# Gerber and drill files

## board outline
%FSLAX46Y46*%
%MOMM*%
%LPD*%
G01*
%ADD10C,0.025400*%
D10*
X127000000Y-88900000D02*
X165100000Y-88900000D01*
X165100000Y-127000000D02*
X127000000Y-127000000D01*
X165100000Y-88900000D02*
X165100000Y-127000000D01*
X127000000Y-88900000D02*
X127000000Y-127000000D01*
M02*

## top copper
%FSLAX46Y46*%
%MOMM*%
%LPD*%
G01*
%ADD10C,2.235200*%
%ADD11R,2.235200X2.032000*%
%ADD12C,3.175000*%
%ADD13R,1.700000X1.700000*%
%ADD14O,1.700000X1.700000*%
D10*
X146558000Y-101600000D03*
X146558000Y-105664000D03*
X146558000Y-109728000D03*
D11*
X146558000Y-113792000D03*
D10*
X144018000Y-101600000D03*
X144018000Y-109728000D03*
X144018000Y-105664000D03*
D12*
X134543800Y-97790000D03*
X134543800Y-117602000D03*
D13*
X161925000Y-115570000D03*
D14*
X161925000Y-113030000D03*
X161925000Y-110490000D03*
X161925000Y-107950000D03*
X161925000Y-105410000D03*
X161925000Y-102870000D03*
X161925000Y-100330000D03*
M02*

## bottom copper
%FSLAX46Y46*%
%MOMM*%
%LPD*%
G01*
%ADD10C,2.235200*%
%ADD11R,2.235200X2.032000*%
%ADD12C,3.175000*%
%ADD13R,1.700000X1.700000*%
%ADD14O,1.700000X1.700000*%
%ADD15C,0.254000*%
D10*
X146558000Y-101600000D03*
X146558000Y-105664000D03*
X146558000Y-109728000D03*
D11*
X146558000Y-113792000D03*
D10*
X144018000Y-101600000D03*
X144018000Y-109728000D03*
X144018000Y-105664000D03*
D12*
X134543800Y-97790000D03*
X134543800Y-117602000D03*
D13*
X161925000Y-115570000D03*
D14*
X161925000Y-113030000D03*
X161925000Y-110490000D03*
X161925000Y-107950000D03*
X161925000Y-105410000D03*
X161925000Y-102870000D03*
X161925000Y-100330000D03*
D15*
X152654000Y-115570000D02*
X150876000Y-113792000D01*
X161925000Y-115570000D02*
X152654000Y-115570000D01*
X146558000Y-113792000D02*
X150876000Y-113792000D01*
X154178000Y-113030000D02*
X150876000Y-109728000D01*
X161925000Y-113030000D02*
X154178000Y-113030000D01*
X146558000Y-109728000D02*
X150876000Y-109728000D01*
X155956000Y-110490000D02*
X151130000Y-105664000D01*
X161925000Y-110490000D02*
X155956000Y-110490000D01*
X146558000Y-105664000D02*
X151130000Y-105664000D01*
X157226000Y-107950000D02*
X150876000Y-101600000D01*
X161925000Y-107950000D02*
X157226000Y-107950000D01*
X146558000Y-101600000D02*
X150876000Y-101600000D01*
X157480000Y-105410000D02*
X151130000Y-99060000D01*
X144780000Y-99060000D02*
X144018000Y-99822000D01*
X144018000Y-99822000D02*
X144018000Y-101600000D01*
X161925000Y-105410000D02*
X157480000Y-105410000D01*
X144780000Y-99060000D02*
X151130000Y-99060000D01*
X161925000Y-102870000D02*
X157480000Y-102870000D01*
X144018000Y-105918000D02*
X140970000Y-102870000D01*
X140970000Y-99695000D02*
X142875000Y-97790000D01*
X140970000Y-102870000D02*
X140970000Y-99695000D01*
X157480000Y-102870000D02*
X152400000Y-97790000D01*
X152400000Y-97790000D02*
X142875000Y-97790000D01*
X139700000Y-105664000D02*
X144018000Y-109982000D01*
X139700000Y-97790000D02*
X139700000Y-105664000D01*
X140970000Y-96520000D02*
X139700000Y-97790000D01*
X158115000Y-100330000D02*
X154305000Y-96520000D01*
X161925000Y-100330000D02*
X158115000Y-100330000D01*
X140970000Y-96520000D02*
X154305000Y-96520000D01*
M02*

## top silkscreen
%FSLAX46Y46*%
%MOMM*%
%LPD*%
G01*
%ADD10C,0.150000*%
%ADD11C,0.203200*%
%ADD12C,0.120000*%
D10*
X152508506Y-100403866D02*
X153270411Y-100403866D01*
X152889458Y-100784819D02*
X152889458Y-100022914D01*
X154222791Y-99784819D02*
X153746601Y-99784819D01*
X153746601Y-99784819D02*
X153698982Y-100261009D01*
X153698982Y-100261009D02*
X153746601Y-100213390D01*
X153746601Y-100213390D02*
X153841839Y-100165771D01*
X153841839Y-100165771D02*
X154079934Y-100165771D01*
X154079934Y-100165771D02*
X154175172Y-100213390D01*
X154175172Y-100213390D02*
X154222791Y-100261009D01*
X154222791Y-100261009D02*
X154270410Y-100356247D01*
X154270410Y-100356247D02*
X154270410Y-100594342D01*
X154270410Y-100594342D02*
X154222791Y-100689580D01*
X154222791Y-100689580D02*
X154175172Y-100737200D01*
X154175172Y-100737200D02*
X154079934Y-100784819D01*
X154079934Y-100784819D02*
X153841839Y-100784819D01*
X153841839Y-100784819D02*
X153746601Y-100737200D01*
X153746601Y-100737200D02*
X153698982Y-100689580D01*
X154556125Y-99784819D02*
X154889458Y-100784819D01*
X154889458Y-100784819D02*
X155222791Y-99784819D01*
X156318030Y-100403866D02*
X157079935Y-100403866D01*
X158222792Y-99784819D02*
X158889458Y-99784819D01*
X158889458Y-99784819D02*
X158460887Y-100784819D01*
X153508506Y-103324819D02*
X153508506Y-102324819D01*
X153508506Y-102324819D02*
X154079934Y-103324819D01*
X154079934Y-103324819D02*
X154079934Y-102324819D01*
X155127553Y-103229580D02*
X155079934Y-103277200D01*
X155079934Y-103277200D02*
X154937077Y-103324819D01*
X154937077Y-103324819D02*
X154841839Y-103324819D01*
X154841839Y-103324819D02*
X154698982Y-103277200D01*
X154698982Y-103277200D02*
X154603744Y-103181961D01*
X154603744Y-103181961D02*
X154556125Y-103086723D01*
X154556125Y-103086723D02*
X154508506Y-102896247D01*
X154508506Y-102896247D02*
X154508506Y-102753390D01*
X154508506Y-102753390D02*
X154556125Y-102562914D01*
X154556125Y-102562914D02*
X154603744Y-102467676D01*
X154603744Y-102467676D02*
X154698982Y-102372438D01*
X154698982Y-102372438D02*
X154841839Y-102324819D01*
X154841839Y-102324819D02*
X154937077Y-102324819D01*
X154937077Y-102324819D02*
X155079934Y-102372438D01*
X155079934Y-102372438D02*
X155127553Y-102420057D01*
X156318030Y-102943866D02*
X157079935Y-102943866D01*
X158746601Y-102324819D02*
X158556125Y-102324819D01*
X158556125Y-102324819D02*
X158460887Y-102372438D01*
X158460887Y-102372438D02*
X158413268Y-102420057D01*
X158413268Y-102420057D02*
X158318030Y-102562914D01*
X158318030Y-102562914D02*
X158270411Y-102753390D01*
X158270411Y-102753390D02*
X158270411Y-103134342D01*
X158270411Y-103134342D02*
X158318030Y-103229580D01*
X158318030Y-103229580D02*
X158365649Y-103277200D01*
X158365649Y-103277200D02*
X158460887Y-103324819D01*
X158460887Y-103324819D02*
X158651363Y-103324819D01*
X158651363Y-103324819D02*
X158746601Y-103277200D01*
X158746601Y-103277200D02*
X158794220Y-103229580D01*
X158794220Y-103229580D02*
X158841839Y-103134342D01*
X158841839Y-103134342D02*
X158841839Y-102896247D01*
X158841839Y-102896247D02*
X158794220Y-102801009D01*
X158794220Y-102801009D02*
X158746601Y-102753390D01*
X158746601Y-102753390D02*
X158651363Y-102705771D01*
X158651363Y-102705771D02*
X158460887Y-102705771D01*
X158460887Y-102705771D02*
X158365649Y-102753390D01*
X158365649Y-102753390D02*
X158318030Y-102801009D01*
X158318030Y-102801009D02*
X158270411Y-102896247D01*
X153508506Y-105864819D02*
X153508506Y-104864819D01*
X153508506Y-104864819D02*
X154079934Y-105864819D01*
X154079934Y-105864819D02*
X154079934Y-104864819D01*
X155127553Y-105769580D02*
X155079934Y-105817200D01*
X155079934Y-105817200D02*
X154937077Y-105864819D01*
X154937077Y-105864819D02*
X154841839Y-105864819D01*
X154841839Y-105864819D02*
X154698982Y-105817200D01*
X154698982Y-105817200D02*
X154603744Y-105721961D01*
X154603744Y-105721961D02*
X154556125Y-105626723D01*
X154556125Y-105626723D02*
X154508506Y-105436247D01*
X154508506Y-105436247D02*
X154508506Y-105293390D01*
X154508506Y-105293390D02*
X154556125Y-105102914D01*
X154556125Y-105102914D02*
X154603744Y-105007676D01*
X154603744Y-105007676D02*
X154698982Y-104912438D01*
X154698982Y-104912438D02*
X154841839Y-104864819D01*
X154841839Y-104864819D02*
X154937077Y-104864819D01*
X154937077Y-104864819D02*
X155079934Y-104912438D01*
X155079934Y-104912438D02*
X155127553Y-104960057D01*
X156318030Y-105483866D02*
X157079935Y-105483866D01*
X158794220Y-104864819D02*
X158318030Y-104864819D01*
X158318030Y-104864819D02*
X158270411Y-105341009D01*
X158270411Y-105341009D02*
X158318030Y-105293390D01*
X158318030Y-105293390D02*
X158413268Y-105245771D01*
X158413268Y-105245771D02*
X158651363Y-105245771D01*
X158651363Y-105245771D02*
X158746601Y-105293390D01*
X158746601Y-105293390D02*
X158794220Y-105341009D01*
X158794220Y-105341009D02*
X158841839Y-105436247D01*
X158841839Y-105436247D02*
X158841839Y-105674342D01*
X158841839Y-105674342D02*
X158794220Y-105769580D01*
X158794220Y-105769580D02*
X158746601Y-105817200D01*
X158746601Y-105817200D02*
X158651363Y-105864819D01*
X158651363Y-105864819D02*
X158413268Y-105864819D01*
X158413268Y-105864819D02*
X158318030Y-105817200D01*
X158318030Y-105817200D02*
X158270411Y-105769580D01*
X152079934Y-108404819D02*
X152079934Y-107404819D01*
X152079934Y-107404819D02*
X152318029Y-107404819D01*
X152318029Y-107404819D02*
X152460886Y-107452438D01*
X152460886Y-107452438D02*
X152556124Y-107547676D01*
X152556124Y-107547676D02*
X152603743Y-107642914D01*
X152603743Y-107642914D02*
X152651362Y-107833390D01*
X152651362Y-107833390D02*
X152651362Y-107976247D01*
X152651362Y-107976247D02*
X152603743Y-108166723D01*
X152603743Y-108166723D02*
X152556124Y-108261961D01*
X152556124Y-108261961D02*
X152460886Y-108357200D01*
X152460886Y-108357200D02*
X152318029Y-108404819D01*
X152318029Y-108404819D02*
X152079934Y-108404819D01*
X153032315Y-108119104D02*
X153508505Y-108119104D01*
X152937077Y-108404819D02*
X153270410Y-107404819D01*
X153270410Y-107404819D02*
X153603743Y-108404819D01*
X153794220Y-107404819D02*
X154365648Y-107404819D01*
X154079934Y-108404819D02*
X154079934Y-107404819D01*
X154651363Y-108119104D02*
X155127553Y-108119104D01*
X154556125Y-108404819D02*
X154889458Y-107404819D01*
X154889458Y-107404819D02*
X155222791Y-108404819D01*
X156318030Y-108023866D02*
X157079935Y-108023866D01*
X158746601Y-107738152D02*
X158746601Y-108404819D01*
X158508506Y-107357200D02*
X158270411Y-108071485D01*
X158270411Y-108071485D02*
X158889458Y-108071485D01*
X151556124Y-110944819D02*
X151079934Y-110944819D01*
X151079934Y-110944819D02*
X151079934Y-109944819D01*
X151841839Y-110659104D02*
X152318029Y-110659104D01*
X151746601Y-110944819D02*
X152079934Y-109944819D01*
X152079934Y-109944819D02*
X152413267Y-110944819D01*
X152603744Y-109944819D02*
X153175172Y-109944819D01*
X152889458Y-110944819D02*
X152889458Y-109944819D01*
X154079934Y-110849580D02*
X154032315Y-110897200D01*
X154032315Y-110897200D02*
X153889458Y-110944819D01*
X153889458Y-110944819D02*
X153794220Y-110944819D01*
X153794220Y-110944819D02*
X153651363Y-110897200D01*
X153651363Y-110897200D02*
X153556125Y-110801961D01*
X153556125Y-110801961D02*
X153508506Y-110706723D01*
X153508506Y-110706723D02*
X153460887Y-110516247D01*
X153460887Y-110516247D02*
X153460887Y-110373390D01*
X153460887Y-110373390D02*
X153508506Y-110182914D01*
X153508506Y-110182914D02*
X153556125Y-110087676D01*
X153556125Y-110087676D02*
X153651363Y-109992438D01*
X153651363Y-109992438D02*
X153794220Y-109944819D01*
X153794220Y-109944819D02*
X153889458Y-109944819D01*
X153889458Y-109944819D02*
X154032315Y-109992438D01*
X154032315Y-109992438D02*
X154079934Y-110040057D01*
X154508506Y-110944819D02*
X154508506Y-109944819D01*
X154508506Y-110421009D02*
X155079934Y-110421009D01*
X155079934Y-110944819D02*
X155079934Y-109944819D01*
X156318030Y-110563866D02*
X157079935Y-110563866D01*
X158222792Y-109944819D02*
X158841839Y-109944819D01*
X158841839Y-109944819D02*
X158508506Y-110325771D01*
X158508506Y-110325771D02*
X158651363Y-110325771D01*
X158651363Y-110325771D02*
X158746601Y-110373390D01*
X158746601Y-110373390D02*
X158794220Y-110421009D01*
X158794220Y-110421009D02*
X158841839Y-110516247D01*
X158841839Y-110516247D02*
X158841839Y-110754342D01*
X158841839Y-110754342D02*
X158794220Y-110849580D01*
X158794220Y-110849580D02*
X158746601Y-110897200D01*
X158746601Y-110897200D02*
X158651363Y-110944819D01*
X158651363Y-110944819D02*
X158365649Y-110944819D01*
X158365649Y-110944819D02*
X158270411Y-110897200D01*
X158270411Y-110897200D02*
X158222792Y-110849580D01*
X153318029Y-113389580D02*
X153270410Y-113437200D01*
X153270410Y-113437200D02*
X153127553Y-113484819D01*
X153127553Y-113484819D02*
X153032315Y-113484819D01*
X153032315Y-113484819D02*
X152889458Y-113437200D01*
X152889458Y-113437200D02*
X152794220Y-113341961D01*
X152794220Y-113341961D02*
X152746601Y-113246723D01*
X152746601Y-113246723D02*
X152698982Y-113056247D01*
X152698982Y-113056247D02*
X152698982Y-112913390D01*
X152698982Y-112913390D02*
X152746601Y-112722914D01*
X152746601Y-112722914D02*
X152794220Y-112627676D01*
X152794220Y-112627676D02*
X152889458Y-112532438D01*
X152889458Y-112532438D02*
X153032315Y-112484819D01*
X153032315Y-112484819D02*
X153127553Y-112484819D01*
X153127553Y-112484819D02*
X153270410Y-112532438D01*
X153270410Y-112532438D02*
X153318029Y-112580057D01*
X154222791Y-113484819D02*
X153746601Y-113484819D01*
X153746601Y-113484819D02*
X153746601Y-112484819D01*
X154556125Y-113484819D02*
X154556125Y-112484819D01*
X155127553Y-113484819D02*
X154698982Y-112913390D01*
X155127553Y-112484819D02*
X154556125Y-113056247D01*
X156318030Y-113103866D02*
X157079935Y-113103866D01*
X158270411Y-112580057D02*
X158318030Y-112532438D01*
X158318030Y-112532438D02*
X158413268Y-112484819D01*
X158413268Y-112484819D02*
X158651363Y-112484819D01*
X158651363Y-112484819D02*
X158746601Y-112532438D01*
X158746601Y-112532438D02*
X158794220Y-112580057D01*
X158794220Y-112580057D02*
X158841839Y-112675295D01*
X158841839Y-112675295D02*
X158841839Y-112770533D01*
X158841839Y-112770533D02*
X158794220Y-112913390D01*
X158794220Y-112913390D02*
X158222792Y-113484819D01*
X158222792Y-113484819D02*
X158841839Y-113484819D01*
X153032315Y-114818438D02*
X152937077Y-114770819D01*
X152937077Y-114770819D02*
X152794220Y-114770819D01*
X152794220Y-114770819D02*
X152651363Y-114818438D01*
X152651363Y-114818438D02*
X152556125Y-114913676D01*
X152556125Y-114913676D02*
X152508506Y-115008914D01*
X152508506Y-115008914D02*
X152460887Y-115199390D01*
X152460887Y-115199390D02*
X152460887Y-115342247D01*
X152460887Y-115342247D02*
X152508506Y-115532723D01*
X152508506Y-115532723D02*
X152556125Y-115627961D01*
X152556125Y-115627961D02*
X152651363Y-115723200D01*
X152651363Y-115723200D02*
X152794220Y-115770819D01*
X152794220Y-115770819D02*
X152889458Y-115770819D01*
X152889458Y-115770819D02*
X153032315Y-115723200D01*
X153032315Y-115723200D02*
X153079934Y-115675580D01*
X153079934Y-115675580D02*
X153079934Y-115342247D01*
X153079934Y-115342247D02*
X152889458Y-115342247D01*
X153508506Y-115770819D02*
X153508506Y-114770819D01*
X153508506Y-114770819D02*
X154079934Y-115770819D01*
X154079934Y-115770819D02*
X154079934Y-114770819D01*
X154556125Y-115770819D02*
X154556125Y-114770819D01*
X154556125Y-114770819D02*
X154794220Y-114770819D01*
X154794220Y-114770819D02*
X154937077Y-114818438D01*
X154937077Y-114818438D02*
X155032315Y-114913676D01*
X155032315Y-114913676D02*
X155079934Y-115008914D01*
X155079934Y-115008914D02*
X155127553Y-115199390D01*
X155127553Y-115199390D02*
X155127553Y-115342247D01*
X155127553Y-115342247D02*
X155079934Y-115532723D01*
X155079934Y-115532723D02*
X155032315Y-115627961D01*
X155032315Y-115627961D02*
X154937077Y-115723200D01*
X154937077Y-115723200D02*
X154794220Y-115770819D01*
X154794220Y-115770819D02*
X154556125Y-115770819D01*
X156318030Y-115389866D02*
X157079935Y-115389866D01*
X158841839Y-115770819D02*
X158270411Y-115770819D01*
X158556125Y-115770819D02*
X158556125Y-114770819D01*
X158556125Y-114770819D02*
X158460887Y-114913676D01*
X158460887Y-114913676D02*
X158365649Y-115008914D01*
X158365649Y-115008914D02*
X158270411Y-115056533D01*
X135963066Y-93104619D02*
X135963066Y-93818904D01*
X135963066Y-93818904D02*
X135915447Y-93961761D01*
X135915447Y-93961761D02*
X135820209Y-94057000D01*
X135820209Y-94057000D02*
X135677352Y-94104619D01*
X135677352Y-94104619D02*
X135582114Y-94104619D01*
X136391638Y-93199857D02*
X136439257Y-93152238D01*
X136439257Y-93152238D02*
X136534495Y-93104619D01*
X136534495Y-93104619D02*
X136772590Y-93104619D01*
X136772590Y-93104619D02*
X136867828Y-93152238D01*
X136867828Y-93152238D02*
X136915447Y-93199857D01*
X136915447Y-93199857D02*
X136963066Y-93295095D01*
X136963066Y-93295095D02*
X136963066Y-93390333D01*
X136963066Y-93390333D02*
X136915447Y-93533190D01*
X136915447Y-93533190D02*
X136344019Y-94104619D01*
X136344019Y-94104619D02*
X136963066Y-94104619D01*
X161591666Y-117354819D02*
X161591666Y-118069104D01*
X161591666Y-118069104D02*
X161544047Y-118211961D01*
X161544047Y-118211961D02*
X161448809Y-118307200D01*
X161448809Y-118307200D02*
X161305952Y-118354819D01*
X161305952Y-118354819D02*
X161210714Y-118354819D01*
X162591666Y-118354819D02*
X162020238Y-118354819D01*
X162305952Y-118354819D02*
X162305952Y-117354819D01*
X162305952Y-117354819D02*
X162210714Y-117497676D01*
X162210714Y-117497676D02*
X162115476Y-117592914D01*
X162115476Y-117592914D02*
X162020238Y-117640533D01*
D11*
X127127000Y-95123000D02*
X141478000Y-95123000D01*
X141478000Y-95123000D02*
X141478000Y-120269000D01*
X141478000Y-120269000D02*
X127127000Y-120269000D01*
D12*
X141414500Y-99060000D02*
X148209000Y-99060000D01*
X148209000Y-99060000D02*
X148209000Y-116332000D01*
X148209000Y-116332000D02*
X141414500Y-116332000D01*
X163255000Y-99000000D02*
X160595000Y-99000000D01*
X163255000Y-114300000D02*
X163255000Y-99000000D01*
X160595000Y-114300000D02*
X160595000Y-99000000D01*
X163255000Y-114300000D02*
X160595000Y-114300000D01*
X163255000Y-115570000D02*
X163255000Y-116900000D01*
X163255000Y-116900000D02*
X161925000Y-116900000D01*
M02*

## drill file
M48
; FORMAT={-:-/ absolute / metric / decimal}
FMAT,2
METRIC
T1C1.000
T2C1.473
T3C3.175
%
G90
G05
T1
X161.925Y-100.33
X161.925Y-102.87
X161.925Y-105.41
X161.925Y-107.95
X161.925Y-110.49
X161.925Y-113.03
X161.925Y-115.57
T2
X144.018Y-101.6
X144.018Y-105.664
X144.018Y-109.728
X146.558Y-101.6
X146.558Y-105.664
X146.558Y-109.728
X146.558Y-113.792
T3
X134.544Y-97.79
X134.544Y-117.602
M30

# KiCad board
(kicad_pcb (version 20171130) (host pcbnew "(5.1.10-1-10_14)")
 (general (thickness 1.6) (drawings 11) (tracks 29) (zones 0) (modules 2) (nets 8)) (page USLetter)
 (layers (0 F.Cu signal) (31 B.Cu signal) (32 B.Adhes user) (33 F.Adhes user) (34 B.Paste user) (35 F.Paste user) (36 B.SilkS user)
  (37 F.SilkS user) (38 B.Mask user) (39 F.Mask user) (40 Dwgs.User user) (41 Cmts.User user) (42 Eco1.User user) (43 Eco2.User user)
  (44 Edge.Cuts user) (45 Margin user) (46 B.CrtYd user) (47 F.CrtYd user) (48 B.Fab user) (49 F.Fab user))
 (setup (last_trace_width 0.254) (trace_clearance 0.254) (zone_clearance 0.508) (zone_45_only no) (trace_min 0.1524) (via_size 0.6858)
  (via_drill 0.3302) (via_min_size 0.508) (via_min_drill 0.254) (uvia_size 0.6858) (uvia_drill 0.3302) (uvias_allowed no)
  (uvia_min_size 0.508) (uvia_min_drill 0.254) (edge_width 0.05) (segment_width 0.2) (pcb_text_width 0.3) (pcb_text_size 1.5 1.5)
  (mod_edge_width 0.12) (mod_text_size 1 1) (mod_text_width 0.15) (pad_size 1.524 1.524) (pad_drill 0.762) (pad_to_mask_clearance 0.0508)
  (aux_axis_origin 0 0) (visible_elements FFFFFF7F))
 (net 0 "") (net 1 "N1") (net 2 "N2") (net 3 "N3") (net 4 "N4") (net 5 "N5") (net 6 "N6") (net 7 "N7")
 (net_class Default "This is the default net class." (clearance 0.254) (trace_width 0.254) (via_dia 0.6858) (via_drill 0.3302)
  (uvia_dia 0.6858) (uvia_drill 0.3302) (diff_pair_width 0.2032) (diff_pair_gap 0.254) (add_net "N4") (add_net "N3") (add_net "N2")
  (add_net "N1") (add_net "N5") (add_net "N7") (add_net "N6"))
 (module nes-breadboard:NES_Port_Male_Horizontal (layer F.Cu) (at 147.574 107.696)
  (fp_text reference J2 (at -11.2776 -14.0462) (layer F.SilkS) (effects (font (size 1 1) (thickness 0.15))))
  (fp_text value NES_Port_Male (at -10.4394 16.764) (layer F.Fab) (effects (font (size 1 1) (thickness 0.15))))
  (fp_line (start -20.447 -12.573) (end -6.096 -12.573) (layer F.SilkS) (width 0.2032))
  (fp_line (start -6.096 -12.573) (end -6.096 12.573) (layer F.SilkS) (width 0.2032))
  (fp_line (start -6.096 12.573) (end -20.447 12.573) (layer F.SilkS) (width 0.2032))
  (fp_line (start -6.1595 -8.636) (end 0.635 -8.636) (layer F.SilkS) (width 0.12))
  (fp_line (start 0.635 -8.636) (end 0.635 8.636) (layer F.SilkS) (width 0.12))
  (fp_line (start 0.635 8.636) (end -6.1595 8.636) (layer F.SilkS) (width 0.12))
  (pad 4 thru_hole circle (at -1.016 -6.096) (size 2.2352 2.2352) (drill 1.4732) (layers *.Cu *.Mask) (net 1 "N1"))
  (pad 3 thru_hole circle (at -1.016 -2.032) (size 2.2352 2.2352) (drill 1.4732) (layers *.Cu *.Mask) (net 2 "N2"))
  (pad 2 thru_hole circle (at -1.016 2.032) (size 2.2352 2.2352) (drill 1.4732) (layers *.Cu *.Mask) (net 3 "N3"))
  (pad 1 thru_hole rect (at -1.016 6.096) (size 2.2352 2.032) (drill 1.4732) (layers *.Cu *.Mask) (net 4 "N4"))
  (pad 5 thru_hole circle (at -3.556 -6.096) (size 2.2352 2.2352) (drill 1.4732) (layers *.Cu *.Mask) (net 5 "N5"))
  (pad 7 thru_hole circle (at -3.556 2.032) (size 2.2352 2.2352) (drill 1.4732) (layers *.Cu *.Mask) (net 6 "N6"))
  (pad 6 thru_hole circle (at -3.556 -2.032) (size 2.2352 2.2352) (drill 1.4732) (layers *.Cu *.Mask) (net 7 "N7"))
  (pad "" thru_hole circle (at -13.0302 -9.906) (size 3.175 3.175) (drill 3.175) (layers *.Cu *.Mask))
  (pad "" thru_hole circle (at -13.0302 9.906) (size 3.175 3.175) (drill 3.175) (layers *.Cu *.Mask)))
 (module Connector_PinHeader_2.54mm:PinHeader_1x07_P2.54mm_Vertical (layer F.Cu) (at 161.925 115.57 180)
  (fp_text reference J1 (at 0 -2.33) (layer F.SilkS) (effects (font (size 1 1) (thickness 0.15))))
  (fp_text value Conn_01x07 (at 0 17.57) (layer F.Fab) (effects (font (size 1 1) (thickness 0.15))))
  (fp_line (start -1.33 16.57) (end 1.33 16.57) (layer F.SilkS) (width 0.12))
  (fp_line (start -1.33 1.27) (end -1.33 16.57) (layer F.SilkS) (width 0.12))
  (fp_line (start 1.33 1.27) (end 1.33 16.57) (layer F.SilkS) (width 0.12))
  (fp_line (start -1.33 1.27) (end 1.33 1.27) (layer F.SilkS) (width 0.12))
  (fp_line (start -1.33 0) (end -1.33 -1.33) (layer F.SilkS) (width 0.12))
  (fp_line (start -1.33 -1.33) (end 0 -1.33) (layer F.SilkS) (width 0.12))
  (pad 1 thru_hole rect (at 0 0 180) (size 1.7 1.7) (drill 1) (layers *.Cu *.Mask) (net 4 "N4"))
  (pad 2 thru_hole oval (at 0 2.54 180) (size 1.7 1.7) (drill 1) (layers *.Cu *.Mask) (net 3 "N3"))
  (pad 3 thru_hole oval (at 0 5.08 180) (size 1.7 1.7) (drill 1) (layers *.Cu *.Mask) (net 2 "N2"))
  (pad 4 thru_hole oval (at 0 7.62 180) (size 1.7 1.7) (drill 1) (layers *.Cu *.Mask) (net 1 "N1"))
  (pad 5 thru_hole oval (at 0 10.16 180) (size 1.7 1.7) (drill 1) (layers *.Cu *.Mask) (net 5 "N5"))
  (pad 6 thru_hole oval (at 0 12.7 180) (size 1.7 1.7) (drill 1) (layers *.Cu *.Mask) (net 7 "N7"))
  (pad 7 thru_hole oval (at 0 15.24 180) (size 1.7 1.7) (drill 1) (layers *.Cu *.Mask) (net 6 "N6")))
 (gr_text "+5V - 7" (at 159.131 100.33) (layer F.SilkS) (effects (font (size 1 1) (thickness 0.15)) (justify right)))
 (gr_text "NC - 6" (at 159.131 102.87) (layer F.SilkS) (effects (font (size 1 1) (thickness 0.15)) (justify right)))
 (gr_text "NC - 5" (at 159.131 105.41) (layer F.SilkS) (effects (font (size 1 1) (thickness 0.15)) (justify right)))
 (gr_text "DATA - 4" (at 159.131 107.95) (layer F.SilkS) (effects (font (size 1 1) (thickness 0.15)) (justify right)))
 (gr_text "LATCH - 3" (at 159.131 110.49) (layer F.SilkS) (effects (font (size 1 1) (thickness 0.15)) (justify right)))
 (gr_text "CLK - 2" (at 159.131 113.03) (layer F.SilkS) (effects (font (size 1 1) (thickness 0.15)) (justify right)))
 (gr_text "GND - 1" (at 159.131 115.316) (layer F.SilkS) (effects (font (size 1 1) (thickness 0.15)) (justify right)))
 (gr_line (start 127 88.9) (end 165.1 88.9) (layer Edge.Cuts) (width 0.0254))
 (gr_line (start 165.1 127) (end 127 127) (layer Edge.Cuts) (width 0.0254))
 (gr_line (start 165.1 88.9) (end 165.1 127) (layer Edge.Cuts) (width 0.0254))
 (gr_line (start 127 88.9) (end 127 127) (layer Edge.Cuts) (width 0.0254))
 (segment (start 152.654 115.57) (end 150.876 113.792) (width 0.254) (layer B.Cu) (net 4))
 (segment (start 161.925 115.57) (end 152.654 115.57) (width 0.254) (layer B.Cu) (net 4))
 (segment (start 146.558 113.792) (end 150.876 113.792) (width 0.254) (layer B.Cu) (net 4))
 (segment (start 154.178 113.03) (end 150.876 109.728) (width 0.254) (layer B.Cu) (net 3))
 (segment (start 161.925 113.03) (end 154.178 113.03) (width 0.254) (layer B.Cu) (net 3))
 (segment (start 146.558 109.728) (end 150.876 109.728) (width 0.254) (layer B.Cu) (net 3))
 (segment (start 155.956 110.49) (end 151.13 105.664) (width 0.254) (layer B.Cu) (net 2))
 (segment (start 161.925 110.49) (end 155.956 110.49) (width 0.254) (layer B.Cu) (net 2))
 (segment (start 146.558 105.664) (end 151.13 105.664) (width 0.254) (layer B.Cu) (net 2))
 (segment (start 157.226 107.95) (end 150.876 101.6) (width 0.254) (layer B.Cu) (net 1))
 (segment (start 161.925 107.95) (end 157.226 107.95) (width 0.254) (layer B.Cu) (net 1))
 (segment (start 146.558 101.6) (end 150.876 101.6) (width 0.254) (layer B.Cu) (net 1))
 (segment (start 157.48 105.41) (end 151.13 99.06) (width 0.254) (layer B.Cu) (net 5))
 (segment (start 144.78 99.06) (end 144.018 99.822) (width 0.254) (layer B.Cu) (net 5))
 (segment (start 144.018 99.822) (end 144.018 101.6) (width 0.254) (layer B.Cu) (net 5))
 (segment (start 161.925 105.41) (end 157.48 105.41) (width 0.254) (layer B.Cu) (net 5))
 (segment (start 144.78 99.06) (end 151.13 99.06) (width 0.254) (layer B.Cu) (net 5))
 (segment (start 161.925 102.87) (end 157.48 102.87) (width 0.254) (layer B.Cu) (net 7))
 (segment (start 144.018 105.918) (end 140.97 102.87) (width 0.254) (layer B.Cu) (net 7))
 (segment (start 140.97 99.695) (end 142.875 97.79) (width 0.254) (layer B.Cu) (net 7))
 (segment (start 140.97 102.87) (end 140.97 99.695) (width 0.254) (layer B.Cu) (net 7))
 (segment (start 157.48 102.87) (end 152.4 97.79) (width 0.254) (layer B.Cu) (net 7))
 (segment (start 152.4 97.79) (end 142.875 97.79) (width 0.254) (layer B.Cu) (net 7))
 (segment (start 139.7 105.664) (end 144.018 109.982) (width 0.254) (layer B.Cu) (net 6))
 (segment (start 139.7 97.79) (end 139.7 105.664) (width 0.254) (layer B.Cu) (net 6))
 (segment (start 140.97 96.52) (end 139.7 97.79) (width 0.254) (layer B.Cu) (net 6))
 (segment (start 158.115 100.33) (end 154.305 96.52) (width 0.254) (layer B.Cu) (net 6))
 (segment (start 161.925 100.33) (end 158.115 100.33) (width 0.254) (layer B.Cu) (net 6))
 (segment (start 140.97 96.52) (end 154.305 96.52) (width 0.254) (layer B.Cu) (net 6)))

